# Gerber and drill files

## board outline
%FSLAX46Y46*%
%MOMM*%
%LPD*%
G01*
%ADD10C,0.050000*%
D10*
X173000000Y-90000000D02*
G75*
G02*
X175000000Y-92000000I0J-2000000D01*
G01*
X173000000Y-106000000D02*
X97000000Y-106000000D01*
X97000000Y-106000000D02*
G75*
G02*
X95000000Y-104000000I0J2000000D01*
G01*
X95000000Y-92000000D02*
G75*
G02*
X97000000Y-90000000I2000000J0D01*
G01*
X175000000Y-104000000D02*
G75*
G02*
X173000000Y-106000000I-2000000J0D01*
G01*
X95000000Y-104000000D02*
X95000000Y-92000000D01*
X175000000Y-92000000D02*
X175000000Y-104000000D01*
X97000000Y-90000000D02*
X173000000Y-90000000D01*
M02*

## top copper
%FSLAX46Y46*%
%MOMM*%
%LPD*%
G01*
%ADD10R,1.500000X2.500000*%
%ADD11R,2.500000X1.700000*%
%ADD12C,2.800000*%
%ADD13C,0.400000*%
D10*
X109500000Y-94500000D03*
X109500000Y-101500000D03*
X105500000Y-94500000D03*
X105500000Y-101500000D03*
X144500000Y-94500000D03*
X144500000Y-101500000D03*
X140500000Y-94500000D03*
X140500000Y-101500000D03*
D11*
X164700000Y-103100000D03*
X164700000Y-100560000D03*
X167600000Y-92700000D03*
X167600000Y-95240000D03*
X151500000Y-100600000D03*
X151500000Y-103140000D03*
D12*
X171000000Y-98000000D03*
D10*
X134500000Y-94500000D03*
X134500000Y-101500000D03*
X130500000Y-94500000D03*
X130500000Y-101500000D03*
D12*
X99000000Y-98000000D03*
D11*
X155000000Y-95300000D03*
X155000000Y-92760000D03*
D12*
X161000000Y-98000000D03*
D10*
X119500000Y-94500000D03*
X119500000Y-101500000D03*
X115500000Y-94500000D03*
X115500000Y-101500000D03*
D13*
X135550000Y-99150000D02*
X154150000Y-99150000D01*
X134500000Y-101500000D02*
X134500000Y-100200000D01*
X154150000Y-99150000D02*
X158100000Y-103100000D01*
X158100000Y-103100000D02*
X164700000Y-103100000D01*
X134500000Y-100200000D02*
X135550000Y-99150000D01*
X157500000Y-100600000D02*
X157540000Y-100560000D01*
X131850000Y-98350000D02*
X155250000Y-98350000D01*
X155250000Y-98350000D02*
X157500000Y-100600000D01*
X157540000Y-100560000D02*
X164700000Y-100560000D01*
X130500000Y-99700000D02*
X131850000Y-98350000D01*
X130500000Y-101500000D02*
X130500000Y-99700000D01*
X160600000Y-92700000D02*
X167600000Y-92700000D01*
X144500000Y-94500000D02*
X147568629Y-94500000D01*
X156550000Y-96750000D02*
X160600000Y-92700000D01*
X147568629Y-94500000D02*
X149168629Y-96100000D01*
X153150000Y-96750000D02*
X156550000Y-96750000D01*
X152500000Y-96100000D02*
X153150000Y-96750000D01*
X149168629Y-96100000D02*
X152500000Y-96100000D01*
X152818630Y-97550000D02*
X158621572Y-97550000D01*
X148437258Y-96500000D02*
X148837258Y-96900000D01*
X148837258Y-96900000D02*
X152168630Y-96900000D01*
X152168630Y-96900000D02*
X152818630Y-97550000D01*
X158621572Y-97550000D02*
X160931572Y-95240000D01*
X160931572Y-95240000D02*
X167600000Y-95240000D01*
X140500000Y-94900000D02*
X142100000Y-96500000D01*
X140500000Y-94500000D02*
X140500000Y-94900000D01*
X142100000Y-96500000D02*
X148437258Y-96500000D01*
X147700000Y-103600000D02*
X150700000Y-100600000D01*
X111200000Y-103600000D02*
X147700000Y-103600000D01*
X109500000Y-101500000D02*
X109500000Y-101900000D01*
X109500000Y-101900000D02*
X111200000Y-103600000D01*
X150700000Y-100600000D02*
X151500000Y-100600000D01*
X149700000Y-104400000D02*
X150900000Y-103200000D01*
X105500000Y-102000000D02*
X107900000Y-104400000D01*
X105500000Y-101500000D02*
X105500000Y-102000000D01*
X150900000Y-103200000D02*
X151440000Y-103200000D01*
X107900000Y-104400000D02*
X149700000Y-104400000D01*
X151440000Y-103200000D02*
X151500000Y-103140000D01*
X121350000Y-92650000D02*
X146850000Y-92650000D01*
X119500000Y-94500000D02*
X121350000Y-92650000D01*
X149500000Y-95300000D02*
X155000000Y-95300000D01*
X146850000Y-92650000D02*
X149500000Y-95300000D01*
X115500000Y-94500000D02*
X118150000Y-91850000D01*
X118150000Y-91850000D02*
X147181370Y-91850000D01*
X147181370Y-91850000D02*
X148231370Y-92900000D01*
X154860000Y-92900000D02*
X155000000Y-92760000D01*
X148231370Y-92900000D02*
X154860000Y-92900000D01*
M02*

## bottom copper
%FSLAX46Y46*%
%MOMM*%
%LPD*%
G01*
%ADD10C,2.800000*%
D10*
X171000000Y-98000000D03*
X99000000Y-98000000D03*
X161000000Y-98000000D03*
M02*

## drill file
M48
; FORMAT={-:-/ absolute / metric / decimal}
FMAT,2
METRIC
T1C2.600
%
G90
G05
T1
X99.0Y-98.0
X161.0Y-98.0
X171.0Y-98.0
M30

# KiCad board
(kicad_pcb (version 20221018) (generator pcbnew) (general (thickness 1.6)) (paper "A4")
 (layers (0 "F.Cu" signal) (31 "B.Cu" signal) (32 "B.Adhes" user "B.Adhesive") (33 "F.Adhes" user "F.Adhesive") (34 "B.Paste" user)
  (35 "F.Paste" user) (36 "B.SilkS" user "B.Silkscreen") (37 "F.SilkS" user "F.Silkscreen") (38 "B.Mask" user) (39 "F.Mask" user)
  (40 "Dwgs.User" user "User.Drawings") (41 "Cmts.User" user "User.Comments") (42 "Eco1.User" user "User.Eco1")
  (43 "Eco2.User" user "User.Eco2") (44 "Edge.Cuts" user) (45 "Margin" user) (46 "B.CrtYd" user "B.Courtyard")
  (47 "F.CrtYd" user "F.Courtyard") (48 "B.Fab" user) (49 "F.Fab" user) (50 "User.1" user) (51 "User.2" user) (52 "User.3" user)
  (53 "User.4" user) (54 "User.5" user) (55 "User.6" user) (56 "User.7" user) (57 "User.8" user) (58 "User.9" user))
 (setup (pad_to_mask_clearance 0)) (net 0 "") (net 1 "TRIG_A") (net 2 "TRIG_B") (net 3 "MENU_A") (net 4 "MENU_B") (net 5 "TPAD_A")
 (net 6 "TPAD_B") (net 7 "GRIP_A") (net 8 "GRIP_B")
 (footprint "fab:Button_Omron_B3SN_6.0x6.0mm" (layer "F.Cu") (at 107.5 98 -90)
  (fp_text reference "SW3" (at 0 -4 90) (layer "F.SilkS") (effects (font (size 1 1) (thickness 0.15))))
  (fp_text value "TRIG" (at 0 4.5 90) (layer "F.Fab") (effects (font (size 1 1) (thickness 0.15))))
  (pad "1" smd rect (at -3.5 -2 270) (size 2.5 1.5) (layers "F.Cu" "F.Paste" "F.Mask") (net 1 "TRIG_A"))
  (pad "1" smd rect (at 3.5 -2 270) (size 2.5 1.5) (layers "F.Cu" "F.Paste" "F.Mask") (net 1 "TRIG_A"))
  (pad "2" smd rect (at -3.5 2 270) (size 2.5 1.5) (layers "F.Cu" "F.Paste" "F.Mask") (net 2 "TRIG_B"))
  (pad "2" smd rect (at 3.5 2 270) (size 2.5 1.5) (layers "F.Cu" "F.Paste" "F.Mask") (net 2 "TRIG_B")))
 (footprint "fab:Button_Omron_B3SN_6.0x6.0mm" (layer "F.Cu") (at 142.5 98 -90)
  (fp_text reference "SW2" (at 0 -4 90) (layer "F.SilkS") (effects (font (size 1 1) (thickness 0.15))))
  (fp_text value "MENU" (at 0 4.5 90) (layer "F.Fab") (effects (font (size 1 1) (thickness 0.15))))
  (pad "1" smd rect (at -3.5 -2 270) (size 2.5 1.5) (layers "F.Cu" "F.Paste" "F.Mask") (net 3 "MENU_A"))
  (pad "1" smd rect (at 3.5 -2 270) (size 2.5 1.5) (layers "F.Cu" "F.Paste" "F.Mask") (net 3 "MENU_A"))
  (pad "2" smd rect (at -3.5 2 270) (size 2.5 1.5) (layers "F.Cu" "F.Paste" "F.Mask") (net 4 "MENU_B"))
  (pad "2" smd rect (at 3.5 2 270) (size 2.5 1.5) (layers "F.Cu" "F.Paste" "F.Mask") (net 4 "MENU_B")))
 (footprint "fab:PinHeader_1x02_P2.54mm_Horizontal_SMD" (layer "F.Cu") (at 164.7 103.1 180)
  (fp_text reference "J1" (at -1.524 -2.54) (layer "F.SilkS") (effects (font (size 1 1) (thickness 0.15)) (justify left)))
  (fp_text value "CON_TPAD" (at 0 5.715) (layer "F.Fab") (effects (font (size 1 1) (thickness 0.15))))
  (pad "1" smd rect (at 0 0 180) (size 2.5 1.7) (layers "F.Cu" "F.Paste" "F.Mask") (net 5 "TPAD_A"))
  (pad "2" smd rect (at 0 2.54 180) (size 2.5 1.7) (layers "F.Cu" "F.Paste" "F.Mask") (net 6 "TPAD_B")))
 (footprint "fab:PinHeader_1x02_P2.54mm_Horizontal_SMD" (layer "F.Cu") (at 167.6 92.7)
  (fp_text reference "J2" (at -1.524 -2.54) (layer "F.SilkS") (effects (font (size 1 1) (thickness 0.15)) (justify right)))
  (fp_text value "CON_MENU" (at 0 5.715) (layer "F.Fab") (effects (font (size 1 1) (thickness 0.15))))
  (pad "1" smd rect (at 0 0) (size 2.5 1.7) (layers "F.Cu" "F.Paste" "F.Mask") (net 3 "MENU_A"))
  (pad "2" smd rect (at 0 2.54) (size 2.5 1.7) (layers "F.Cu" "F.Paste" "F.Mask") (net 4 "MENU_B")))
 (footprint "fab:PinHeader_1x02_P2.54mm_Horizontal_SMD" (layer "F.Cu") (at 151.5 100.6)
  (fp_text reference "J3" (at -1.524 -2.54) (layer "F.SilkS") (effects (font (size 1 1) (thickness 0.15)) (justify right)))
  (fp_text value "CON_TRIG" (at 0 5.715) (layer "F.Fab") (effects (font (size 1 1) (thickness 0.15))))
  (pad "1" smd rect (at 0 0) (size 2.5 1.7) (layers "F.Cu" "F.Paste" "F.Mask") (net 1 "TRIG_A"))
  (pad "2" smd rect (at 0 2.54) (size 2.5 1.7) (layers "F.Cu" "F.Paste" "F.Mask") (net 2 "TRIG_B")))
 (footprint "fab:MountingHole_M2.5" (layer "F.Cu") (at 171 98 -90)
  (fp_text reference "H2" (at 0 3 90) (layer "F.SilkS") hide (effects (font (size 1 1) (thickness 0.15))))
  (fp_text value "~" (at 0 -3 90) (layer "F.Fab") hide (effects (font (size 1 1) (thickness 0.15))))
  (pad "" thru_hole circle (at 0 0 270) (size 2.8 2.8) (drill 2.6) (layers "*.Cu" "*.Mask")))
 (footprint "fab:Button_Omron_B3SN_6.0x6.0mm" (layer "F.Cu") (at 132.5 98 -90)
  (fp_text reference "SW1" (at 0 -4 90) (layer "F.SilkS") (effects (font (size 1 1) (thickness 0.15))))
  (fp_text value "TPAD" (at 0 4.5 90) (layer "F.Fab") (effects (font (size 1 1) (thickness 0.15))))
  (pad "1" smd rect (at -3.5 -2 270) (size 2.5 1.5) (layers "F.Cu" "F.Paste" "F.Mask") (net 5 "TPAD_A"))
  (pad "1" smd rect (at 3.5 -2 270) (size 2.5 1.5) (layers "F.Cu" "F.Paste" "F.Mask") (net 5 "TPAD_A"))
  (pad "2" smd rect (at -3.5 2 270) (size 2.5 1.5) (layers "F.Cu" "F.Paste" "F.Mask") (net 6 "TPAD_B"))
  (pad "2" smd rect (at 3.5 2 270) (size 2.5 1.5) (layers "F.Cu" "F.Paste" "F.Mask") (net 6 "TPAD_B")))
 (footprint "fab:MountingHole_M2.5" (layer "F.Cu") (at 99 98 -90)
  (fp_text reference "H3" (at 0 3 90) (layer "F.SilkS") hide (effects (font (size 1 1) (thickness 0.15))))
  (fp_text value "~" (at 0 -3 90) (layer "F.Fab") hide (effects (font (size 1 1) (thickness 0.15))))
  (pad "" thru_hole circle (at 0 0 270) (size 2.8 2.8) (drill 2.6) (layers "*.Cu" "*.Mask")))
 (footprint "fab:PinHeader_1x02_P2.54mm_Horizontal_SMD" (layer "F.Cu") (at 155 95.3 180)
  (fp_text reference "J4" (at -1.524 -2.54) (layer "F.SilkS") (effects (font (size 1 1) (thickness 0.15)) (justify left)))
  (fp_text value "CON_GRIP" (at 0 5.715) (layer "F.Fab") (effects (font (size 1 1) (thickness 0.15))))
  (pad "1" smd rect (at 0 0 180) (size 2.5 1.7) (layers "F.Cu" "F.Paste" "F.Mask") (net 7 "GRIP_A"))
  (pad "2" smd rect (at 0 2.54 180) (size 2.5 1.7) (layers "F.Cu" "F.Paste" "F.Mask") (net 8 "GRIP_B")))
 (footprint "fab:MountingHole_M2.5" (layer "F.Cu") (at 161 98 -90)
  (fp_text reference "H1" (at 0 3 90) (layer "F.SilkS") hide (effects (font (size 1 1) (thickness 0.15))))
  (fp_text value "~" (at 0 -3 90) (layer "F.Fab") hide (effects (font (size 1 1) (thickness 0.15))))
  (pad "" thru_hole circle (at 0 0 270) (size 2.8 2.8) (drill 2.6) (layers "*.Cu" "*.Mask")))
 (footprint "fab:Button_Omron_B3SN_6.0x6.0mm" (layer "F.Cu") (at 117.5 98 -90)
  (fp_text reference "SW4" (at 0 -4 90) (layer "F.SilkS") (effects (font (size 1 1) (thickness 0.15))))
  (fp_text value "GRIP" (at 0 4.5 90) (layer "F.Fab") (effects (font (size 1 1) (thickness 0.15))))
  (pad "1" smd rect (at -3.5 -2 270) (size 2.5 1.5) (layers "F.Cu" "F.Paste" "F.Mask") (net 7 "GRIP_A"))
  (pad "1" smd rect (at 3.5 -2 270) (size 2.5 1.5) (layers "F.Cu" "F.Paste" "F.Mask") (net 7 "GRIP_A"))
  (pad "2" smd rect (at -3.5 2 270) (size 2.5 1.5) (layers "F.Cu" "F.Paste" "F.Mask") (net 8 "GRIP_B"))
  (pad "2" smd rect (at 3.5 2 270) (size 2.5 1.5) (layers "F.Cu" "F.Paste" "F.Mask") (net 8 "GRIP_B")))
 (gr_arc (start 173 90) (mid 174.414214 90.585786) (end 175 92) (stroke (width 0.05) (type default)) (layer "Edge.Cuts"))
 (gr_line (start 173 106) (end 97 106) (stroke (width 0.05) (type default)) (layer "Edge.Cuts"))
 (gr_arc (start 97 106) (mid 95.585786 105.414214) (end 95 104) (stroke (width 0.05) (type default)) (layer "Edge.Cuts"))
 (gr_arc (start 95 92) (mid 95.585786 90.585786) (end 97 90) (stroke (width 0.05) (type default)) (layer "Edge.Cuts"))
 (gr_arc (start 175 104) (mid 174.414214 105.414214) (end 173 106) (stroke (width 0.05) (type default)) (layer "Edge.Cuts"))
 (gr_line (start 95 104) (end 95 92) (stroke (width 0.05) (type default)) (layer "Edge.Cuts"))
 (gr_line (start 175 92) (end 175 104) (stroke (width 0.05) (type default)) (layer "Edge.Cuts"))
 (gr_line (start 97 90) (end 173 90) (stroke (width 0.05) (type default)) (layer "Edge.Cuts"))
 (segment (start 135.55 99.15) (end 154.15 99.15) (width 0.4) (layer "F.Cu") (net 5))
 (segment (start 134.5 101.5) (end 134.5 100.2) (width 0.4) (layer "F.Cu") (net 5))
 (segment (start 154.15 99.15) (end 158.1 103.1) (width 0.4) (layer "F.Cu") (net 5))
 (segment (start 158.1 103.1) (end 164.7 103.1) (width 0.4) (layer "F.Cu") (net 5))
 (segment (start 134.5 100.2) (end 135.55 99.15) (width 0.4) (layer "F.Cu") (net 5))
 (segment (start 157.5 100.6) (end 157.54 100.56) (width 0.4) (layer "F.Cu") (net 6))
 (segment (start 131.85 98.35) (end 155.25 98.35) (width 0.4) (layer "F.Cu") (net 6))
 (segment (start 155.25 98.35) (end 157.5 100.6) (width 0.4) (layer "F.Cu") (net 6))
 (segment (start 157.54 100.56) (end 164.7 100.56) (width 0.4) (layer "F.Cu") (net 6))
 (segment (start 130.5 99.7) (end 131.85 98.35) (width 0.4) (layer "F.Cu") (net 6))
 (segment (start 130.5 101.5) (end 130.5 99.7) (width 0.4) (layer "F.Cu") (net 6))
 (segment (start 160.6 92.7) (end 167.6 92.7) (width 0.4) (layer "F.Cu") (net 3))
 (segment (start 144.5 94.5) (end 147.568629 94.5) (width 0.4) (layer "F.Cu") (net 3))
 (segment (start 156.55 96.75) (end 160.6 92.7) (width 0.4) (layer "F.Cu") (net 3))
 (segment (start 147.568629 94.5) (end 149.168629 96.1) (width 0.4) (layer "F.Cu") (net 3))
 (segment (start 153.15 96.75) (end 156.55 96.75) (width 0.4) (layer "F.Cu") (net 3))
 (segment (start 152.5 96.1) (end 153.15 96.75) (width 0.4) (layer "F.Cu") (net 3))
 (segment (start 149.168629 96.1) (end 152.5 96.1) (width 0.4) (layer "F.Cu") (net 3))
 (segment (start 152.81863 97.55) (end 158.621572 97.55) (width 0.4) (layer "F.Cu") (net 4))
 (segment (start 148.437258 96.5) (end 148.837258 96.9) (width 0.4) (layer "F.Cu") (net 4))
 (segment (start 148.837258 96.9) (end 152.16863 96.9) (width 0.4) (layer "F.Cu") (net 4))
 (segment (start 152.16863 96.9) (end 152.81863 97.55) (width 0.4) (layer "F.Cu") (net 4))
 (segment (start 158.621572 97.55) (end 160.931572 95.24) (width 0.4) (layer "F.Cu") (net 4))
 (segment (start 160.931572 95.24) (end 167.6 95.24) (width 0.4) (layer "F.Cu") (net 4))
 (segment (start 140.5 94.9) (end 142.1 96.5) (width 0.4) (layer "F.Cu") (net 4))
 (segment (start 140.5 94.5) (end 140.5 94.9) (width 0.4) (layer "F.Cu") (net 4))
 (segment (start 142.1 96.5) (end 148.437258 96.5) (width 0.4) (layer "F.Cu") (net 4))
 (segment (start 147.7 103.6) (end 150.7 100.6) (width 0.4) (layer "F.Cu") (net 1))
 (segment (start 111.2 103.6) (end 147.7 103.6) (width 0.4) (layer "F.Cu") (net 1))
 (segment (start 109.5 101.5) (end 109.5 101.9) (width 0.4) (layer "F.Cu") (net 1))
 (segment (start 109.5 101.9) (end 111.2 103.6) (width 0.4) (layer "F.Cu") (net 1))
 (segment (start 150.7 100.6) (end 151.5 100.6) (width 0.4) (layer "F.Cu") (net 1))
 (segment (start 149.7 104.4) (end 150.9 103.2) (width 0.4) (layer "F.Cu") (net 2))
 (segment (start 105.5 102) (end 107.9 104.4) (width 0.4) (layer "F.Cu") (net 2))
 (segment (start 105.5 101.5) (end 105.5 102) (width 0.4) (layer "F.Cu") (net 2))
 (segment (start 150.9 103.2) (end 151.44 103.2) (width 0.4) (layer "F.Cu") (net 2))
 (segment (start 107.9 104.4) (end 149.7 104.4) (width 0.4) (layer "F.Cu") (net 2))
 (segment (start 151.44 103.2) (end 151.5 103.14) (width 0.4) (layer "F.Cu") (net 2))
 (segment (start 121.35 92.65) (end 146.85 92.65) (width 0.4) (layer "F.Cu") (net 7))
 (segment (start 119.5 94.5) (end 121.35 92.65) (width 0.4) (layer "F.Cu") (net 7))
 (segment (start 149.5 95.3) (end 155 95.3) (width 0.4) (layer "F.Cu") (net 7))
 (segment (start 146.85 92.65) (end 149.5 95.3) (width 0.4) (layer "F.Cu") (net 7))
 (segment (start 115.5 94.5) (end 118.15 91.85) (width 0.4) (layer "F.Cu") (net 8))
 (segment (start 118.15 91.85) (end 147.18137 91.85) (width 0.4) (layer "F.Cu") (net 8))
 (segment (start 147.18137 91.85) (end 148.23137 92.9) (width 0.4) (layer "F.Cu") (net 8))
 (segment (start 154.86 92.9) (end 155 92.76) (width 0.4) (layer "F.Cu") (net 8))
 (segment (start 148.23137 92.9) (end 154.86 92.9) (width 0.4) (layer "F.Cu") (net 8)))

